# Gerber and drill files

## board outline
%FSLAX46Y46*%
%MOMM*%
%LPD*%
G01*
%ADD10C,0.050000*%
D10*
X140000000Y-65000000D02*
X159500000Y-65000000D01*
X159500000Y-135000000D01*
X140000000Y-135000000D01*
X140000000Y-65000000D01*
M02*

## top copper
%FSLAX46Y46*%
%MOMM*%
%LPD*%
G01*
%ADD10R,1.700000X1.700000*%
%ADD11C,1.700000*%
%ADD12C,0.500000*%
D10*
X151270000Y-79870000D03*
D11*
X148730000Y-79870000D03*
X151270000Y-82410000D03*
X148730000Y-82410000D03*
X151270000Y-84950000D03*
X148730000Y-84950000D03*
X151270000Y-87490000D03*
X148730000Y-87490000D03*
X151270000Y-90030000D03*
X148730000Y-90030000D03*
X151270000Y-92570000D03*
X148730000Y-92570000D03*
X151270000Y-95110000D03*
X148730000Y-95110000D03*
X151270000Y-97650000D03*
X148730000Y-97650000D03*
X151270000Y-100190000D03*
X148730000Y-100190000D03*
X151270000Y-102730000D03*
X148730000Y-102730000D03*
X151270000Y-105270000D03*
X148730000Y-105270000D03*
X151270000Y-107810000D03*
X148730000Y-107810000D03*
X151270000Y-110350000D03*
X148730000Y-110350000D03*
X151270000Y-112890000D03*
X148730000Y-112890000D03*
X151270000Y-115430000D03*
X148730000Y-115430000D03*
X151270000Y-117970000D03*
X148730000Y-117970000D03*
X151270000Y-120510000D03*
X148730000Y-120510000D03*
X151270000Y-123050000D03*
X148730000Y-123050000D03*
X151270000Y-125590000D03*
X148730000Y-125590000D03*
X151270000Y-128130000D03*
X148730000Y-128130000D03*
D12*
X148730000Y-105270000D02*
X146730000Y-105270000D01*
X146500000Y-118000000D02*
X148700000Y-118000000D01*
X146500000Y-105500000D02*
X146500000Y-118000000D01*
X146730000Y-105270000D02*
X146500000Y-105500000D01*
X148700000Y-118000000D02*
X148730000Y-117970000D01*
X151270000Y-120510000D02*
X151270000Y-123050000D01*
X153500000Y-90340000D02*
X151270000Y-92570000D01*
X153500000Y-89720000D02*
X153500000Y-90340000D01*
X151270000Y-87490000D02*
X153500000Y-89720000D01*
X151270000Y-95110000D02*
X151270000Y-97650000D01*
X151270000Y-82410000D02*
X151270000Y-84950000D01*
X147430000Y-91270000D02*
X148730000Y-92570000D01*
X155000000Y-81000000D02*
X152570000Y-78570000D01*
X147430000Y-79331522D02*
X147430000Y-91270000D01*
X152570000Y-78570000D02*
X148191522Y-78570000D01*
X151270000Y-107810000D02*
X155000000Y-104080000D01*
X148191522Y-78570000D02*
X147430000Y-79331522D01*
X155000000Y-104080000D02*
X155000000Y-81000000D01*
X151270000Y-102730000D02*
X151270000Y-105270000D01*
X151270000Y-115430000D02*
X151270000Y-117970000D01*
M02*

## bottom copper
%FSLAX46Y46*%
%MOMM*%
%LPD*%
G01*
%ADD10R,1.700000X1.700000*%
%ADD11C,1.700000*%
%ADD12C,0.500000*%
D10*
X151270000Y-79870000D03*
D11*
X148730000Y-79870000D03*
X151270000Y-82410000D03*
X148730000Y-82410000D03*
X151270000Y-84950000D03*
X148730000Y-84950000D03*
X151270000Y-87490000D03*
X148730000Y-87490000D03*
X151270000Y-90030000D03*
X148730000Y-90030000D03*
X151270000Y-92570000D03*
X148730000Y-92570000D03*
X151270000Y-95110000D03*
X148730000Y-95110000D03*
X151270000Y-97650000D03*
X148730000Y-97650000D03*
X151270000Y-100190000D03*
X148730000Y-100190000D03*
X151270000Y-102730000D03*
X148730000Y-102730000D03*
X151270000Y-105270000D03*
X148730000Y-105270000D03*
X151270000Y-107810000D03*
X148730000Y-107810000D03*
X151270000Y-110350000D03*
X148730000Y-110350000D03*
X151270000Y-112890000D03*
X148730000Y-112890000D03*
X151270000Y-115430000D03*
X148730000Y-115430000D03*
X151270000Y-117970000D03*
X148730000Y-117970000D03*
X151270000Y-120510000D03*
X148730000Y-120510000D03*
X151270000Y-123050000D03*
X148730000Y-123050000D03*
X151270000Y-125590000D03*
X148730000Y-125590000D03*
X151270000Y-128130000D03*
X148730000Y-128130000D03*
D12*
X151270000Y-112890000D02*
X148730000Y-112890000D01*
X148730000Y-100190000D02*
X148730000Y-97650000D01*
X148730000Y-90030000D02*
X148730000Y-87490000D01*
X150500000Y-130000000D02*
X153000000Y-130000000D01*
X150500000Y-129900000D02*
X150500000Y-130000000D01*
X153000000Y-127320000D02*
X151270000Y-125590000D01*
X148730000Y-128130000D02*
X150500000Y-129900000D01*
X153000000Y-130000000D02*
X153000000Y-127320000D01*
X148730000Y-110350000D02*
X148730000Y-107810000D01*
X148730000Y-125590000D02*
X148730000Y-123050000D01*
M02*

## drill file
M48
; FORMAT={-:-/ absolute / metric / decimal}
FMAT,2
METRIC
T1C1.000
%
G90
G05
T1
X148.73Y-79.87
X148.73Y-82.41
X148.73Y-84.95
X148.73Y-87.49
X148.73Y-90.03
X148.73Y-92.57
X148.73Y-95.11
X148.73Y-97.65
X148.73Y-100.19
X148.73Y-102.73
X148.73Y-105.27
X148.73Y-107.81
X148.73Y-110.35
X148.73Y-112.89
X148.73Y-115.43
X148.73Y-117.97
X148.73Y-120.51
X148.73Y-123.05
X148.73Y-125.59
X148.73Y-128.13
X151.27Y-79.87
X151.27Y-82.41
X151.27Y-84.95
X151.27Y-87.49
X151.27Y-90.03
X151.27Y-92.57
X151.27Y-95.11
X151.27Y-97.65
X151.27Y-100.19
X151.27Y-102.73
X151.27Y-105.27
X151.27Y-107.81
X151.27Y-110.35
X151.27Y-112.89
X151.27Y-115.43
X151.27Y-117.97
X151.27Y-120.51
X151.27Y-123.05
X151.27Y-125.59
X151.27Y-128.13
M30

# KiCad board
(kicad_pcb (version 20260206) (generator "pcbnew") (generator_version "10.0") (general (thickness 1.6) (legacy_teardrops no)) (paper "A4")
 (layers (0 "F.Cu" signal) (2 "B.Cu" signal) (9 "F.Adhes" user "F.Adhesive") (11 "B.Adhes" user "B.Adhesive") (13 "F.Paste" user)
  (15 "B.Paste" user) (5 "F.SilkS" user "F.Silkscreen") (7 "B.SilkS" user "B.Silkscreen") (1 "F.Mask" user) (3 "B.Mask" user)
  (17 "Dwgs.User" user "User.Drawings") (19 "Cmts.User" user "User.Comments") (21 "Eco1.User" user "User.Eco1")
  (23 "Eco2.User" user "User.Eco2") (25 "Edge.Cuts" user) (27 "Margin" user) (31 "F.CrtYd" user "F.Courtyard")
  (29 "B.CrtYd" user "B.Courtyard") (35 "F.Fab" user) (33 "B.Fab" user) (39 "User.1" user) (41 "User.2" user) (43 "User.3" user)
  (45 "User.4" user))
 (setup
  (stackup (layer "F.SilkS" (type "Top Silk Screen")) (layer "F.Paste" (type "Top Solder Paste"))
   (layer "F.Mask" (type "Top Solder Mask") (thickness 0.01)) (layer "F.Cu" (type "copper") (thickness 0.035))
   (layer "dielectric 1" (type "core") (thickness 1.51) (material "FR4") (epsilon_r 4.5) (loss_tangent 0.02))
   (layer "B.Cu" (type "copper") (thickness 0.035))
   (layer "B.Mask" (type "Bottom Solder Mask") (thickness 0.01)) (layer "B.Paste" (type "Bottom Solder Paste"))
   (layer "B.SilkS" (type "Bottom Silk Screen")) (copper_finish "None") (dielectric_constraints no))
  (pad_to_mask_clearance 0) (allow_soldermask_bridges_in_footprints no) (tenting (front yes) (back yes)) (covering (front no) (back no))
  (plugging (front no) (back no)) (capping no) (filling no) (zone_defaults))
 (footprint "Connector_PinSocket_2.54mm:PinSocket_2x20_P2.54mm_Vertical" (layer "F.Cu") (at 151.27 79.87)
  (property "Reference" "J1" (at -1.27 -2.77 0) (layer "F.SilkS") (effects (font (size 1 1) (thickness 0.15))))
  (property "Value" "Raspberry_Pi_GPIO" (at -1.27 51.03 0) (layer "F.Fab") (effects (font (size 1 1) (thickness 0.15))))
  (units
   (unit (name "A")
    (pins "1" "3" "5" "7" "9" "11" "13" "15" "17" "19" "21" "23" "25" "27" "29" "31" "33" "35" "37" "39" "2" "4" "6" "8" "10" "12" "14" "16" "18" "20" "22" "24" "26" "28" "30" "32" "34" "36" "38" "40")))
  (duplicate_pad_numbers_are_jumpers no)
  (pad "1" thru_hole rect (at 0 0) (size 1.7 1.7) (drill 1) (layers "*.Cu" "*.Mask") (remove_unused_layers no)
   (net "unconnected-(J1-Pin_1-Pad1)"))
  (pad "2" thru_hole circle (at -2.54 0) (size 1.7 1.7) (drill 1) (layers "*.Cu" "*.Mask") (remove_unused_layers no)
   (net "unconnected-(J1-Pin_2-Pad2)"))
  (pad "3" thru_hole circle (at 0 2.54) (size 1.7 1.7) (drill 1) (layers "*.Cu" "*.Mask") (remove_unused_layers no) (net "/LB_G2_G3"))
  (pad "4" thru_hole circle (at -2.54 2.54) (size 1.7 1.7) (drill 1) (layers "*.Cu" "*.Mask") (remove_unused_layers no)
   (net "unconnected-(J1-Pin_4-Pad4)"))
  (pad "5" thru_hole circle (at 0 5.08) (size 1.7 1.7) (drill 1) (layers "*.Cu" "*.Mask") (remove_unused_layers no) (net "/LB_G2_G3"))
  (pad "6" thru_hole circle (at -2.54 5.08) (size 1.7 1.7) (drill 1) (layers "*.Cu" "*.Mask") (remove_unused_layers no)
   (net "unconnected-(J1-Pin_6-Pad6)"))
  (pad "7" thru_hole circle (at 0 7.62) (size 1.7 1.7) (drill 1) (layers "*.Cu" "*.Mask") (remove_unused_layers no) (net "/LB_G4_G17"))
  (pad "8" thru_hole circle (at -2.54 7.62) (size 1.7 1.7) (drill 1) (layers "*.Cu" "*.Mask") (remove_unused_layers no) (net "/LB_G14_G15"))
  (pad "9" thru_hole circle (at 0 10.16) (size 1.7 1.7) (drill 1) (layers "*.Cu" "*.Mask") (remove_unused_layers no)
   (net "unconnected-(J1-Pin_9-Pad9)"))
  (pad "10" thru_hole circle (at -2.54 10.16) (size 1.7 1.7) (drill 1) (layers "*.Cu" "*.Mask") (remove_unused_layers no)
   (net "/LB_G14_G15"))
  (pad "11" thru_hole circle (at 0 12.7) (size 1.7 1.7) (drill 1) (layers "*.Cu" "*.Mask") (remove_unused_layers no) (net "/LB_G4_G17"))
  (pad "12" thru_hole circle (at -2.54 12.7) (size 1.7 1.7) (drill 1) (layers "*.Cu" "*.Mask") (remove_unused_layers no) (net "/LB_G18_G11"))
  (pad "13" thru_hole circle (at 0 15.24) (size 1.7 1.7) (drill 1) (layers "*.Cu" "*.Mask") (remove_unused_layers no) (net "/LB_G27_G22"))
  (pad "14" thru_hole circle (at -2.54 15.24) (size 1.7 1.7) (drill 1) (layers "*.Cu" "*.Mask") (remove_unused_layers no)
   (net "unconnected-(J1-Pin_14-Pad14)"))
  (pad "15" thru_hole circle (at 0 17.78) (size 1.7 1.7) (drill 1) (layers "*.Cu" "*.Mask") (remove_unused_layers no) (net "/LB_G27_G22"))
  (pad "16" thru_hole circle (at -2.54 17.78) (size 1.7 1.7) (drill 1) (layers "*.Cu" "*.Mask") (remove_unused_layers no)
   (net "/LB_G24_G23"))
  (pad "17" thru_hole circle (at 0 20.32) (size 1.7 1.7) (drill 1) (layers "*.Cu" "*.Mask") (remove_unused_layers no)
   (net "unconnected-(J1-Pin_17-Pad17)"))
  (pad "18" thru_hole circle (at -2.54 20.32) (size 1.7 1.7) (drill 1) (layers "*.Cu" "*.Mask") (remove_unused_layers no)
   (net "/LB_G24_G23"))
  (pad "19" thru_hole circle (at 0 22.86) (size 1.7 1.7) (drill 1) (layers "*.Cu" "*.Mask") (remove_unused_layers no) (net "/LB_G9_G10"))
  (pad "20" thru_hole circle (at -2.54 22.86) (size 1.7 1.7) (drill 1) (layers "*.Cu" "*.Mask") (remove_unused_layers no)
   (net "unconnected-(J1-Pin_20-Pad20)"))
  (pad "21" thru_hole circle (at 0 25.4) (size 1.7 1.7) (drill 1) (layers "*.Cu" "*.Mask") (remove_unused_layers no) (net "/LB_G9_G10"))
  (pad "22" thru_hole circle (at -2.54 25.4) (size 1.7 1.7) (drill 1) (layers "*.Cu" "*.Mask") (remove_unused_layers no) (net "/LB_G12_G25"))
  (pad "23" thru_hole circle (at 0 27.94) (size 1.7 1.7) (drill 1) (layers "*.Cu" "*.Mask") (remove_unused_layers no) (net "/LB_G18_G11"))
  (pad "24" thru_hole circle (at -2.54 27.94) (size 1.7 1.7) (drill 1) (layers "*.Cu" "*.Mask") (remove_unused_layers no) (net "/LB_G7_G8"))
  (pad "25" thru_hole circle (at 0 30.48) (size 1.7 1.7) (drill 1) (layers "*.Cu" "*.Mask") (remove_unused_layers no)
   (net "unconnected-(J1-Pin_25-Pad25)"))
  (pad "26" thru_hole circle (at -2.54 30.48) (size 1.7 1.7) (drill 1) (layers "*.Cu" "*.Mask") (remove_unused_layers no) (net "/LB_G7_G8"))
  (pad "27" thru_hole circle (at 0 33.02) (size 1.7 1.7) (drill 1) (layers "*.Cu" "*.Mask") (remove_unused_layers no) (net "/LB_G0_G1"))
  (pad "28" thru_hole circle (at -2.54 33.02) (size 1.7 1.7) (drill 1) (layers "*.Cu" "*.Mask") (remove_unused_layers no) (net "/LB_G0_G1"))
  (pad "29" thru_hole circle (at 0 35.56) (size 1.7 1.7) (drill 1) (layers "*.Cu" "*.Mask") (remove_unused_layers no) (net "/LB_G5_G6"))
  (pad "30" thru_hole circle (at -2.54 35.56) (size 1.7 1.7) (drill 1) (layers "*.Cu" "*.Mask") (remove_unused_layers no)
   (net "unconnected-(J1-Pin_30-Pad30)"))
  (pad "31" thru_hole circle (at 0 38.1) (size 1.7 1.7) (drill 1) (layers "*.Cu" "*.Mask") (remove_unused_layers no) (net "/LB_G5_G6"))
  (pad "32" thru_hole circle (at -2.54 38.1) (size 1.7 1.7) (drill 1) (layers "*.Cu" "*.Mask") (remove_unused_layers no) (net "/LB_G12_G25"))
  (pad "33" thru_hole circle (at 0 40.64) (size 1.7 1.7) (drill 1) (layers "*.Cu" "*.Mask") (remove_unused_layers no) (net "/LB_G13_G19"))
  (pad "34" thru_hole circle (at -2.54 40.64) (size 1.7 1.7) (drill 1) (layers "*.Cu" "*.Mask") (remove_unused_layers no)
   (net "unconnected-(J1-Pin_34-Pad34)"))
  (pad "35" thru_hole circle (at 0 43.18) (size 1.7 1.7) (drill 1) (layers "*.Cu" "*.Mask") (remove_unused_layers no) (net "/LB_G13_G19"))
  (pad "36" thru_hole circle (at -2.54 43.18) (size 1.7 1.7) (drill 1) (layers "*.Cu" "*.Mask") (remove_unused_layers no)
   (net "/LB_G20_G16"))
  (pad "37" thru_hole circle (at 0 45.72) (size 1.7 1.7) (drill 1) (layers "*.Cu" "*.Mask") (remove_unused_layers no) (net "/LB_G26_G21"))
  (pad "38" thru_hole circle (at -2.54 45.72) (size 1.7 1.7) (drill 1) (layers "*.Cu" "*.Mask") (remove_unused_layers no)
   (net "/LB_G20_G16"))
  (pad "39" thru_hole circle (at 0 48.26) (size 1.7 1.7) (drill 1) (layers "*.Cu" "*.Mask") (remove_unused_layers no)
   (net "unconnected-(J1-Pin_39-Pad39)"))
  (pad "40" thru_hole circle (at -2.54 48.26) (size 1.7 1.7) (drill 1) (layers "*.Cu" "*.Mask") (remove_unused_layers no)
   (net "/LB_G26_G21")))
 (gr_rect (start 140 65) (end 159.5 135) (stroke (width 0.05) (type default)) (fill no) (layer "Edge.Cuts"))
 (segment (start 148.73 105.27) (end 146.73 105.27) (width 0.5) (layer "F.Cu") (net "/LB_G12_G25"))
 (segment (start 146.5 118) (end 148.7 118) (width 0.5) (layer "F.Cu") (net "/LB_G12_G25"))
 (segment (start 146.5 105.5) (end 146.5 118) (width 0.5) (layer "F.Cu") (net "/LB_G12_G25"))
 (segment (start 146.73 105.27) (end 146.5 105.5) (width 0.5) (layer "F.Cu") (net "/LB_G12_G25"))
 (segment (start 148.7 118) (end 148.73 117.97) (width 0.5) (layer "F.Cu") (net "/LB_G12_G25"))
 (segment (start 151.27 112.89) (end 148.73 112.89) (width 0.5) (layer "B.Cu") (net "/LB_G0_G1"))
 (segment (start 148.73 100.19) (end 148.73 97.65) (width 0.5) (layer "B.Cu") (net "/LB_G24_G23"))
 (segment (start 151.27 120.51) (end 151.27 123.05) (width 0.5) (layer "F.Cu") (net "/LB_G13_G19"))
 (segment (start 148.73 90.03) (end 148.73 87.49) (width 0.5) (layer "B.Cu") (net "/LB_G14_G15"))
 (segment (start 153.5 90.34) (end 151.27 92.57) (width 0.5) (layer "F.Cu") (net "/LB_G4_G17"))
 (segment (start 153.5 89.72) (end 153.5 90.34) (width 0.5) (layer "F.Cu") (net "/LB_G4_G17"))
 (segment (start 151.27 87.49) (end 153.5 89.72) (width 0.5) (layer "F.Cu") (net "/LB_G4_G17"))
 (segment (start 150.5 130) (end 153 130) (width 0.5) (layer "B.Cu") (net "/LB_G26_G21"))
 (segment (start 150.5 129.9) (end 150.5 130) (width 0.5) (layer "B.Cu") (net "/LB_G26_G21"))
 (segment (start 153 127.32) (end 151.27 125.59) (width 0.5) (layer "B.Cu") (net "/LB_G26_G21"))
 (segment (start 148.73 128.13) (end 150.5 129.9) (width 0.5) (layer "B.Cu") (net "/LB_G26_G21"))
 (segment (start 153 130) (end 153 127.32) (width 0.5) (layer "B.Cu") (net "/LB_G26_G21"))
 (segment (start 148.73 110.35) (end 148.73 107.81) (width 0.5) (layer "B.Cu") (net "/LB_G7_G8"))
 (segment (start 151.27 95.11) (end 151.27 97.65) (width 0.5) (layer "F.Cu") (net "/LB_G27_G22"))
 (segment (start 151.27 82.41) (end 151.27 84.95) (width 0.5) (layer "F.Cu") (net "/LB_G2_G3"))
 (segment (start 147.43 91.27) (end 148.73 92.57) (width 0.5) (layer "F.Cu") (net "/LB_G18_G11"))
 (segment (start 155 81) (end 152.57 78.57) (width 0.5) (layer "F.Cu") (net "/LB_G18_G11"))
 (segment (start 147.43 79.331522) (end 147.43 91.27) (width 0.5) (layer "F.Cu") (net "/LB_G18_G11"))
 (segment (start 152.57 78.57) (end 148.191522 78.57) (width 0.5) (layer "F.Cu") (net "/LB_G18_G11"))
 (segment (start 151.27 107.81) (end 155 104.08) (width 0.5) (layer "F.Cu") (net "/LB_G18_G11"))
 (segment (start 148.191522 78.57) (end 147.43 79.331522) (width 0.5) (layer "F.Cu") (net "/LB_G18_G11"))
 (segment (start 155 104.08) (end 155 81) (width 0.5) (layer "F.Cu") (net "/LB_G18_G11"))
 (segment (start 151.27 102.73) (end 151.27 105.27) (width 0.5) (layer "F.Cu") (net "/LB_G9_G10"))
 (segment (start 148.73 125.59) (end 148.73 123.05) (width 0.5) (layer "B.Cu") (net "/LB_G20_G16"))
 (segment (start 151.27 115.43) (end 151.27 117.97) (width 0.5) (layer "F.Cu") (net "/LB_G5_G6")))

